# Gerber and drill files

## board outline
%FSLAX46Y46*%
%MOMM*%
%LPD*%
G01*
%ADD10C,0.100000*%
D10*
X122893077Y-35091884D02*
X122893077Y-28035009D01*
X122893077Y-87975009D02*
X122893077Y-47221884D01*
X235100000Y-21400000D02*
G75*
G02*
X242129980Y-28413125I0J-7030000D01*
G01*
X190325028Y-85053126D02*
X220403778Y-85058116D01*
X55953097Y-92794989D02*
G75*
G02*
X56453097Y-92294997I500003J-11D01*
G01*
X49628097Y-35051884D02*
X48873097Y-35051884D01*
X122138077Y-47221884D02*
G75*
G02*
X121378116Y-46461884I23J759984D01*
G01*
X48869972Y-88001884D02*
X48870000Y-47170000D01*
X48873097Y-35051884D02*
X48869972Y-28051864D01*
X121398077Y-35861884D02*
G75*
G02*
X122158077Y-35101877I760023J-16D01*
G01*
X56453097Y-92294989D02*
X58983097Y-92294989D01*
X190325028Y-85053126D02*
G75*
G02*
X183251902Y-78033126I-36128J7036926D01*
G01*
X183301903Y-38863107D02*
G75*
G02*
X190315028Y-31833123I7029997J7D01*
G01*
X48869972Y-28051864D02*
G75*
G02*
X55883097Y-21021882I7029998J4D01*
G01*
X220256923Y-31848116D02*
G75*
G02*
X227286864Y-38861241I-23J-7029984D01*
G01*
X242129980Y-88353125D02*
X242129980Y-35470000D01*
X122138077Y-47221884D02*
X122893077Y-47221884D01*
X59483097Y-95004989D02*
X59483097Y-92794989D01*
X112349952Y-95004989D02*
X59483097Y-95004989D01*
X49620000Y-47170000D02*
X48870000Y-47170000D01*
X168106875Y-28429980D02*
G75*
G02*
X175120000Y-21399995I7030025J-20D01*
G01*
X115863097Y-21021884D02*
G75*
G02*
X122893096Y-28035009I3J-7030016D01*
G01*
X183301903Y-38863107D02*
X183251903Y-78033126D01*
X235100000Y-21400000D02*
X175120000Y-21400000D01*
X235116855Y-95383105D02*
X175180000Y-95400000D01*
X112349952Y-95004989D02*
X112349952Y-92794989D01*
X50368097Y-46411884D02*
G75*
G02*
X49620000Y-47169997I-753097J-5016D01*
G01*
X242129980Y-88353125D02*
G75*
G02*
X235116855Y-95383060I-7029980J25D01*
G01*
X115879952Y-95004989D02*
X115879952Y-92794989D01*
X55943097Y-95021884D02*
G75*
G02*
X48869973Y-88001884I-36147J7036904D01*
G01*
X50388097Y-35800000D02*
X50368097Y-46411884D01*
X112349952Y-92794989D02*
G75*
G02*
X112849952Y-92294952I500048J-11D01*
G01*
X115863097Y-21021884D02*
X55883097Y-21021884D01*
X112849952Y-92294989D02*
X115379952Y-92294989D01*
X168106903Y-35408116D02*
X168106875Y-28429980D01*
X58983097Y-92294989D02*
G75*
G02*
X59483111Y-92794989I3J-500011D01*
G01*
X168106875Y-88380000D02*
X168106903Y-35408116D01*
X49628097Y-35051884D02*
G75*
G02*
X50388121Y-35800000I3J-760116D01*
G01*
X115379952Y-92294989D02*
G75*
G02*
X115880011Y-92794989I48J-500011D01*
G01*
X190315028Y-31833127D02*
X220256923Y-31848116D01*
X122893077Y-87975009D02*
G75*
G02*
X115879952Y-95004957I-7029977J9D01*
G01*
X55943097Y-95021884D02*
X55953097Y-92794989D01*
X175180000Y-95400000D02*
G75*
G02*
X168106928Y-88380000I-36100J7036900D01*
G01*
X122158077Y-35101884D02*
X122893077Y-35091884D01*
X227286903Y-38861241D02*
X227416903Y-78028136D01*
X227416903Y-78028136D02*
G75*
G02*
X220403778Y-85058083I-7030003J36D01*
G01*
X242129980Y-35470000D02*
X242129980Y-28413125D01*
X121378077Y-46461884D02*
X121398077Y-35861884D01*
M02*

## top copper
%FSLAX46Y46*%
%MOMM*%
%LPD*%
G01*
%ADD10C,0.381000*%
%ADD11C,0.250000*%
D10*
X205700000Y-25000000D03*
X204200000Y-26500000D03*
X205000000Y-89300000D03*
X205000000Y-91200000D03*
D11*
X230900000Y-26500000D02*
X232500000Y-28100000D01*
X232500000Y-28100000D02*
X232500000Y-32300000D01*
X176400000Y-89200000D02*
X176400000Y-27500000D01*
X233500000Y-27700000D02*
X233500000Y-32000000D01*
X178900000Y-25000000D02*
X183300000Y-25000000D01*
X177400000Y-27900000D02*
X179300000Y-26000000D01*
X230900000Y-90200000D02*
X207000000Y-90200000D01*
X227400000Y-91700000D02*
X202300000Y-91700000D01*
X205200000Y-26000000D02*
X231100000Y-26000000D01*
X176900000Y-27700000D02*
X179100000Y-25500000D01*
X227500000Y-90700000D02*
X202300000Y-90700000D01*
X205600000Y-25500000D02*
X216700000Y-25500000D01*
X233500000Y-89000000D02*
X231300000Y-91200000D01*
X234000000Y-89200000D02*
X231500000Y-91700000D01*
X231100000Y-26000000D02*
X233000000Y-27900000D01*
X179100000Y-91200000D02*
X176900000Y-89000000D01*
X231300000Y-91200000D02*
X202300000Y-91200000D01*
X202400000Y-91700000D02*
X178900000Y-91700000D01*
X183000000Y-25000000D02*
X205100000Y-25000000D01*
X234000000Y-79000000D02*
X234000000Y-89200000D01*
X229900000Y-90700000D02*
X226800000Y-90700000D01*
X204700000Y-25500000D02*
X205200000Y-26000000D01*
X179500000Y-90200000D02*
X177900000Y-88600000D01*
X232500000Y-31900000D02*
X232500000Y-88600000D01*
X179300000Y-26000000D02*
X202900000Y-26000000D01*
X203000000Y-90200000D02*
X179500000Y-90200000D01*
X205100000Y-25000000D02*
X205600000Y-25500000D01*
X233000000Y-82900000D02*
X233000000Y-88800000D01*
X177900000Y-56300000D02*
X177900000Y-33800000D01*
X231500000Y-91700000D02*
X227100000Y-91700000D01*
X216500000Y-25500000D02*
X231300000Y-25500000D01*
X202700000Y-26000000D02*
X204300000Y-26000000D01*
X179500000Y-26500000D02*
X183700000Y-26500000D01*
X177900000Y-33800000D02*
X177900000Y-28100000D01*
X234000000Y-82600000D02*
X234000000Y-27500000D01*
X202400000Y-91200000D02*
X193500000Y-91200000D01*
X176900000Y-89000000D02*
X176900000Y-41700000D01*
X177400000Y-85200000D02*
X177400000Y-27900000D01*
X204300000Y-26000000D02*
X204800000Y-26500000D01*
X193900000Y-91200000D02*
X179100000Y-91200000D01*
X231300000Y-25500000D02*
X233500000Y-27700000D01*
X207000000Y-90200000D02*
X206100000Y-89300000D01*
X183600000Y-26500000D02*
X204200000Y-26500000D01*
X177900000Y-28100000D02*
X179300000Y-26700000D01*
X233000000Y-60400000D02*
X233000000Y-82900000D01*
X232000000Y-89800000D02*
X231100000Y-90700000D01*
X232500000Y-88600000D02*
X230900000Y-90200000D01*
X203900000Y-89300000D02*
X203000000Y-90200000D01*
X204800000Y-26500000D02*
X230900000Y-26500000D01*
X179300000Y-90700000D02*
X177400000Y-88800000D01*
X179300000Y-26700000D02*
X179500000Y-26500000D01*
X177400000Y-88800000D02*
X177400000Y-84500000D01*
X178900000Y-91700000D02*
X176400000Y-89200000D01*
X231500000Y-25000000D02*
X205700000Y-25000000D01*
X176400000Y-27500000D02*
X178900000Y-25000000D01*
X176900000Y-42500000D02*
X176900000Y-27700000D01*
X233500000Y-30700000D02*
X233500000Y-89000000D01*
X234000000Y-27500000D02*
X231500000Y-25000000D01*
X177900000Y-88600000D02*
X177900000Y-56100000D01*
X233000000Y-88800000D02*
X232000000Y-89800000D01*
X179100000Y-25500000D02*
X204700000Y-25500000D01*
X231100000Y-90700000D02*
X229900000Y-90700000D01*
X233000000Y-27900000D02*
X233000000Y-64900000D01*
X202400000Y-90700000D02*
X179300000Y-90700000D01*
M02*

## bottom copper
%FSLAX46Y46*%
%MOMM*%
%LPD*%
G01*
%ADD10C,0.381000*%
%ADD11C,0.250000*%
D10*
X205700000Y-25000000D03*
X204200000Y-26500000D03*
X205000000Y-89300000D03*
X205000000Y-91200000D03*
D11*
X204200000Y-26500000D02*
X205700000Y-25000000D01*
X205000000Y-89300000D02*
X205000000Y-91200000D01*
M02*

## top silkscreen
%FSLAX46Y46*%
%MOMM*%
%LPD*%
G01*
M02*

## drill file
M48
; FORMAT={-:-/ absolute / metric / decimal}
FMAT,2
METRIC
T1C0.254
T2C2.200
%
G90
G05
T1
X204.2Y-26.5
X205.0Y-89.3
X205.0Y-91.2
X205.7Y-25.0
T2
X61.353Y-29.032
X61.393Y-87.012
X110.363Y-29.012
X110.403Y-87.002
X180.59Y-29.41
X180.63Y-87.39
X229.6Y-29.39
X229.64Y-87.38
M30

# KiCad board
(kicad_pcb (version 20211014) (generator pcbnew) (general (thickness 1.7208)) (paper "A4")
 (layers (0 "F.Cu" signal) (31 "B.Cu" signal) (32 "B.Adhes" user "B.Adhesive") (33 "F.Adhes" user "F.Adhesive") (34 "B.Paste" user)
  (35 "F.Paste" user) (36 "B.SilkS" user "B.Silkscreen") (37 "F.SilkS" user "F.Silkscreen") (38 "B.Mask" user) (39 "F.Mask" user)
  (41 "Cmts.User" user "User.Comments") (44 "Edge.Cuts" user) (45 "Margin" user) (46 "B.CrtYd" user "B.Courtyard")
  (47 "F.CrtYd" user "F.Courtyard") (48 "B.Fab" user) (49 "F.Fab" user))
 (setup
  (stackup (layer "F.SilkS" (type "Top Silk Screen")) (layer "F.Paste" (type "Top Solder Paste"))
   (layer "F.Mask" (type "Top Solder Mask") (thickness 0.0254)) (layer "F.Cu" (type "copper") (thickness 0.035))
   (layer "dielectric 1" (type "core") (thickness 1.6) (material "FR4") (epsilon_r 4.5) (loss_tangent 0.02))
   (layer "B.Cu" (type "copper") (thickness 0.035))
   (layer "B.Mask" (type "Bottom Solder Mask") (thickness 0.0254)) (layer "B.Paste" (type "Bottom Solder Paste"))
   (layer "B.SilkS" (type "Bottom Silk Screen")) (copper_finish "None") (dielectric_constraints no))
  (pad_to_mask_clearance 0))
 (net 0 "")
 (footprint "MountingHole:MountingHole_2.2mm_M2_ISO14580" (layer "F.Cu") (at 61.353097 29.031884)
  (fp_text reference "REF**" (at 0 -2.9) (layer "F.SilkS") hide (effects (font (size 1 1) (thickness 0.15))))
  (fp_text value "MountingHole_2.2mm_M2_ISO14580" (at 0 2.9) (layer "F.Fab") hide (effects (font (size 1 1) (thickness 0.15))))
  (pad "" np_thru_hole circle (at 0 0) (size 2.2 2.2) (drill 2.2) (layers *.Cu *.Mask)))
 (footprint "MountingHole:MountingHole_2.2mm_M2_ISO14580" (layer "F.Cu") (at 61.393097 87.011884)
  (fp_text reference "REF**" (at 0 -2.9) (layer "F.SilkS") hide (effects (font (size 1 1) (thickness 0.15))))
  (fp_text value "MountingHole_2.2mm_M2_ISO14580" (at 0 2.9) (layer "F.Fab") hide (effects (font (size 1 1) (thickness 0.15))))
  (pad "" np_thru_hole circle (at 0 0) (size 2.2 2.2) (drill 2.2) (layers *.Cu *.Mask)))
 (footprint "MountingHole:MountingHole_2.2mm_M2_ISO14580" (layer "F.Cu") (at 110.403097 87.001884)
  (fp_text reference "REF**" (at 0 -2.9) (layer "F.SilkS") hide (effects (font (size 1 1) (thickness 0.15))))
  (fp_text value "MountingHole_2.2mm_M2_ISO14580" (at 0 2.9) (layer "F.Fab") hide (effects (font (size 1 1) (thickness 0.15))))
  (pad "" np_thru_hole circle (at 0 0) (size 2.2 2.2) (drill 2.2) (layers *.Cu *.Mask)))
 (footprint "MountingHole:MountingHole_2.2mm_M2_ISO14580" (layer "F.Cu") (at 229.6 29.39)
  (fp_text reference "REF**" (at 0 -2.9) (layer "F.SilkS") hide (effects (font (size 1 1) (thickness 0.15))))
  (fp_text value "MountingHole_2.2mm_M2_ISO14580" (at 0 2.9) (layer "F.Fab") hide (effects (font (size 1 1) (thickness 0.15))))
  (pad "" np_thru_hole circle (at 0 0) (size 2.2 2.2) (drill 2.2) (layers *.Cu *.Mask)))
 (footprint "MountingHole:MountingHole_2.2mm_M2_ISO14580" (layer "F.Cu") (at 229.64 87.38)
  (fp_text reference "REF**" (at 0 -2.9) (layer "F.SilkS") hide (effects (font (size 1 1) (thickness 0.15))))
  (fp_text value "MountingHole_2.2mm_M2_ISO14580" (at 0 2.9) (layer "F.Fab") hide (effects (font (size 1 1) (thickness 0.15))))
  (pad "" np_thru_hole circle (at 0 0) (size 2.2 2.2) (drill 2.2) (layers *.Cu *.Mask)))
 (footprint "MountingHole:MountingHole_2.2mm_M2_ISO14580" (layer "F.Cu") (at 180.63 87.39)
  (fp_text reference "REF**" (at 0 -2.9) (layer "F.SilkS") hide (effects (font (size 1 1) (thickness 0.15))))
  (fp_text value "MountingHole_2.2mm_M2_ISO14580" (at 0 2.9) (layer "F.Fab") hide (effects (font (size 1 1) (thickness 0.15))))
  (pad "" np_thru_hole circle (at 0 0) (size 2.2 2.2) (drill 2.2) (layers *.Cu *.Mask)))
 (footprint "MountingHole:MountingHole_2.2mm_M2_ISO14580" (layer "F.Cu") (at 110.363097 29.011884)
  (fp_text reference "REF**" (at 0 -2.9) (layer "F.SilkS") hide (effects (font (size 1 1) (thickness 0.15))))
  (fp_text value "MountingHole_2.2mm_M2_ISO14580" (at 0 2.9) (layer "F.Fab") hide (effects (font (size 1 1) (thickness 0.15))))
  (pad "" np_thru_hole circle (at 0 0) (size 2.2 2.2) (drill 2.2) (layers *.Cu *.Mask)))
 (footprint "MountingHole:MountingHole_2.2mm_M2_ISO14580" (layer "F.Cu") (at 180.59 29.41)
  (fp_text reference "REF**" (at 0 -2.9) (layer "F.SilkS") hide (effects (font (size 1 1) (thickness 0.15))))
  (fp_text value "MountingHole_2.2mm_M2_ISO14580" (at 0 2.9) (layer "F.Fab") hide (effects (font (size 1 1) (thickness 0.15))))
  (pad "" np_thru_hole circle (at 0 0) (size 2.2 2.2) (drill 2.2) (layers *.Cu *.Mask)))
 (gr_line (start 122.893077 35.091884) (end 122.893077 28.035009) (layer "Edge.Cuts") (width 0.1))
 (gr_line (start 122.893077 87.975009) (end 122.893077 47.221884) (layer "Edge.Cuts") (width 0.1))
 (gr_arc (start 235.1 21.4) (mid 240.064991 23.453077) (end 242.12998 28.413125) (layer "Edge.Cuts") (width 0.1))
 (gr_line (start 190.325028 85.053126) (end 220.403778 85.058116) (layer "Edge.Cuts") (width 0.1))
 (gr_arc (start 55.953097 92.794989) (mid 56.099544 92.441436) (end 56.453097 92.294989) (layer "Edge.Cuts") (width 0.1))
 (gr_line (start 49.628097 35.051884) (end 48.873097 35.051884) (layer "Edge.Cuts") (width 0.1))
 (gr_arc (start 122.138077 47.221884) (mid 121.600676 46.999285) (end 121.378077 46.461884) (layer "Edge.Cuts") (width 0.1))
 (gr_line (start 48.869972 88.001884) (end 48.87 47.17) (layer "Edge.Cuts") (width 0.1))
 (gr_line (start 48.873097 35.051884) (end 48.869972 28.051864) (layer "Edge.Cuts") (width 0.1))
 (gr_arc (start 121.398077 35.861884) (mid 121.620676 35.324483) (end 122.158077 35.101884) (layer "Edge.Cuts") (width 0.1))
 (gr_line (start 56.453097 92.294989) (end 58.983097 92.294989) (layer "Edge.Cuts") (width 0.1))
 (gr_arc (start 190.325028 85.053126) (mid 185.331764 83.010851) (end 183.251903 78.033126) (layer "Edge.Cuts") (width 0.1))
 (gr_arc (start 183.301903 38.863107) (mid 185.35498 33.898116) (end 190.315028 31.833127) (layer "Edge.Cuts") (width 0.1))
 (gr_arc (start 48.869972 28.051864) (mid 50.923049 23.086873) (end 55.883097 21.021884) (layer "Edge.Cuts") (width 0.1))
 (gr_arc (start 220.256923 31.848116) (mid 225.221914 33.901193) (end 227.286903 38.861241) (layer "Edge.Cuts") (width 0.1))
 (gr_line (start 242.12998 88.353125) (end 242.12998 35.47) (layer "Edge.Cuts") (width 0.1))
 (gr_line (start 122.138077 47.221884) (end 122.893077 47.221884) (layer "Edge.Cuts") (width 0.1))
 (gr_line (start 59.483097 95.004989) (end 59.483097 92.794989) (layer "Edge.Cuts") (width 0.1))
 (gr_line (start 112.349952 95.004989) (end 59.483097 95.004989) (layer "Edge.Cuts") (width 0.1))
 (gr_line (start 49.62 47.17) (end 48.87 47.17) (layer "Edge.Cuts") (width 0.1))
 (gr_arc (start 168.106875 28.42998) (mid 170.159952 23.464989) (end 175.12 21.4) (layer "Edge.Cuts") (width 0.1))
 (gr_arc (start 115.863097 21.021884) (mid 120.828088 23.074961) (end 122.893077 28.035009) (layer "Edge.Cuts") (width 0.1))
 (gr_line (start 183.301903 38.863107) (end 183.251903 78.033126) (layer "Edge.Cuts") (width 0.1))
 (gr_line (start 235.1 21.4) (end 175.12 21.4) (layer "Edge.Cuts") (width 0.1))
 (gr_line (start 235.116855 95.383105) (end 175.18 95.4) (layer "Edge.Cuts") (width 0.1))
 (gr_line (start 112.349952 95.004989) (end 112.349952 92.794989) (layer "Edge.Cuts") (width 0.1))
 (gr_arc (start 50.368097 46.411884) (mid 50.15106 46.945878) (end 49.62 47.17) (layer "Edge.Cuts") (width 0.1))
 (gr_arc (start 242.12998 88.353125) (mid 240.076903 93.318116) (end 235.116855 95.383105) (layer "Edge.Cuts") (width 0.1))
 (gr_line (start 115.879952 95.004989) (end 115.879952 92.794989) (layer "Edge.Cuts") (width 0.1))
 (gr_arc (start 55.943097 95.021884) (mid 50.949833 92.979609) (end 48.869972 88.001884) (layer "Edge.Cuts") (width 0.1))
 (gr_line (start 50.388097 35.8) (end 50.368097 46.411884) (layer "Edge.Cuts") (width 0.1))
 (gr_arc (start 112.349952 92.794989) (mid 112.496399 92.441436) (end 112.849952 92.294989) (layer "Edge.Cuts") (width 0.1))
 (gr_line (start 115.863097 21.021884) (end 55.883097 21.021884) (layer "Edge.Cuts") (width 0.1))
 (gr_line (start 112.849952 92.294989) (end 115.379952 92.294989) (layer "Edge.Cuts") (width 0.1))
 (gr_line (start 168.106903 35.408116) (end 168.106875 28.42998) (layer "Edge.Cuts") (width 0.1))
 (gr_arc (start 58.983097 92.294989) (mid 59.33665 92.441436) (end 59.483097 92.794989) (layer "Edge.Cuts") (width 0.1))
 (gr_line (start 168.106875 88.38) (end 168.106903 35.408116) (layer "Edge.Cuts") (width 0.1))
 (gr_arc (start 49.628097 35.051884) (mid 50.161313 35.270292) (end 50.388097 35.8) (layer "Edge.Cuts") (width 0.1))
 (gr_arc (start 115.379952 92.294989) (mid 115.733505 92.441436) (end 115.879952 92.794989) (layer "Edge.Cuts") (width 0.1))
 (gr_line (start 190.315028 31.833127) (end 220.256923 31.848116) (layer "Edge.Cuts") (width 0.1))
 (gr_arc (start 122.893077 87.975009) (mid 120.84 92.94) (end 115.879952 95.004989) (layer "Edge.Cuts") (width 0.1))
 (gr_line (start 55.943097 95.021884) (end 55.953097 92.794989) (layer "Edge.Cuts") (width 0.1))
 (gr_arc (start 175.18 95.4) (mid 170.186736 93.357725) (end 168.106875 88.38) (layer "Edge.Cuts") (width 0.1))
 (gr_line (start 122.158077 35.101884) (end 122.893077 35.091884) (layer "Edge.Cuts") (width 0.1))
 (gr_line (start 227.286903 38.861241) (end 227.416903 78.028136) (layer "Edge.Cuts") (width 0.1))
 (gr_arc (start 227.416903 78.028136) (mid 225.363826 82.993127) (end 220.403778 85.058116) (layer "Edge.Cuts") (width 0.1))
 (gr_line (start 242.12998 35.47) (end 242.12998 28.413125) (layer "Edge.Cuts") (width 0.1))
 (gr_line (start 121.378077 46.461884) (end 121.398077 35.861884) (layer "Edge.Cuts") (width 0.1))
 (segment (start 230.9 26.5) (end 232.5 28.1) (width 0.25) (layer "F.Cu") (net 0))
 (segment (start 232.5 28.1) (end 232.5 32.3) (width 0.25) (layer "F.Cu") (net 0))
 (segment (start 176.4 89.2) (end 176.4 27.5) (width 0.25) (layer "F.Cu") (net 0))
 (segment (start 233.5 27.7) (end 233.5 32) (width 0.25) (layer "F.Cu") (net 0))
 (segment (start 178.9 25) (end 183.3 25) (width 0.25) (layer "F.Cu") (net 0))
 (segment (start 177.4 27.9) (end 179.3 26) (width 0.25) (layer "F.Cu") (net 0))
 (segment (start 230.9 90.2) (end 207 90.2) (width 0.25) (layer "F.Cu") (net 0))
 (segment (start 227.4 91.7) (end 202.3 91.7) (width 0.25) (layer "F.Cu") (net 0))
 (segment (start 205.2 26) (end 231.1 26) (width 0.25) (layer "F.Cu") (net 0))
 (segment (start 176.9 27.7) (end 179.1 25.5) (width 0.25) (layer "F.Cu") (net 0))
 (segment (start 227.5 90.7) (end 202.3 90.7) (width 0.25) (layer "F.Cu") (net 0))
 (segment (start 205.6 25.5) (end 216.7 25.5) (width 0.25) (layer "F.Cu") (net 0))
 (segment (start 233.5 89) (end 231.3 91.2) (width 0.25) (layer "F.Cu") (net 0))
 (segment (start 234 89.2) (end 231.5 91.7) (width 0.25) (layer "F.Cu") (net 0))
 (segment (start 231.1 26) (end 233 27.9) (width 0.25) (layer "F.Cu") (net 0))
 (segment (start 179.1 91.2) (end 176.9 89) (width 0.25) (layer "F.Cu") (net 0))
 (segment (start 231.3 91.2) (end 202.3 91.2) (width 0.25) (layer "F.Cu") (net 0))
 (segment (start 202.4 91.7) (end 178.9 91.7) (width 0.25) (layer "F.Cu") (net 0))
 (segment (start 183 25) (end 205.1 25) (width 0.25) (layer "F.Cu") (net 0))
 (segment (start 234 79) (end 234 89.2) (width 0.25) (layer "F.Cu") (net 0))
 (segment (start 229.9 90.7) (end 226.8 90.7) (width 0.25) (layer "F.Cu") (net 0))
 (segment (start 204.7 25.5) (end 205.2 26) (width 0.25) (layer "F.Cu") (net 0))
 (segment (start 179.5 90.2) (end 177.9 88.6) (width 0.25) (layer "F.Cu") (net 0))
 (segment (start 232.5 31.9) (end 232.5 88.6) (width 0.25) (layer "F.Cu") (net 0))
 (segment (start 179.3 26) (end 202.9 26) (width 0.25) (layer "F.Cu") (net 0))
 (segment (start 203 90.2) (end 179.5 90.2) (width 0.25) (layer "F.Cu") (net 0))
 (segment (start 205.1 25) (end 205.6 25.5) (width 0.25) (layer "F.Cu") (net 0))
 (segment (start 233 82.9) (end 233 88.8) (width 0.25) (layer "F.Cu") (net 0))
 (segment (start 177.9 56.3) (end 177.9 33.8) (width 0.25) (layer "F.Cu") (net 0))
 (segment (start 231.5 91.7) (end 227.1 91.7) (width 0.25) (layer "F.Cu") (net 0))
 (segment (start 216.5 25.5) (end 231.3 25.5) (width 0.25) (layer "F.Cu") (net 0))
 (segment (start 202.7 26) (end 204.3 26) (width 0.25) (layer "F.Cu") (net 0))
 (segment (start 179.5 26.5) (end 183.7 26.5) (width 0.25) (layer "F.Cu") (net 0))
 (segment (start 177.9 33.8) (end 177.9 28.1) (width 0.25) (layer "F.Cu") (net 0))
 (segment (start 234 82.6) (end 234 27.5) (width 0.25) (layer "F.Cu") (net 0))
 (segment (start 202.4 91.2) (end 193.5 91.2) (width 0.25) (layer "F.Cu") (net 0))
 (segment (start 176.9 89) (end 176.9 41.7) (width 0.25) (layer "F.Cu") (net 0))
 (segment (start 177.4 85.2) (end 177.4 27.9) (width 0.25) (layer "F.Cu") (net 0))
 (segment (start 204.3 26) (end 204.8 26.5) (width 0.25) (layer "F.Cu") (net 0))
 (segment (start 193.9 91.2) (end 179.1 91.2) (width 0.25) (layer "F.Cu") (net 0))
 (segment (start 231.3 25.5) (end 233.5 27.7) (width 0.25) (layer "F.Cu") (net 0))
 (segment (start 207 90.2) (end 206.1 89.3) (width 0.25) (layer "F.Cu") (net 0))
 (segment (start 183.6 26.5) (end 204.2 26.5) (width 0.25) (layer "F.Cu") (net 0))
 (segment (start 177.9 28.1) (end 179.3 26.7) (width 0.25) (layer "F.Cu") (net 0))
 (segment (start 233 60.4) (end 233 82.9) (width 0.25) (layer "F.Cu") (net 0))
 (segment (start 232 89.8) (end 231.1 90.7) (width 0.25) (layer "F.Cu") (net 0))
 (segment (start 232.5 88.6) (end 230.9 90.2) (width 0.25) (layer "F.Cu") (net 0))
 (segment (start 203.9 89.3) (end 203 90.2) (width 0.25) (layer "F.Cu") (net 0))
 (segment (start 204.8 26.5) (end 230.9 26.5) (width 0.25) (layer "F.Cu") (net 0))
 (segment (start 179.3 90.7) (end 177.4 88.8) (width 0.25) (layer "F.Cu") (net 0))
 (segment (start 179.3 26.7) (end 179.5 26.5) (width 0.25) (layer "F.Cu") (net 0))
 (segment (start 177.4 88.8) (end 177.4 84.5) (width 0.25) (layer "F.Cu") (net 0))
 (segment (start 178.9 91.7) (end 176.4 89.2) (width 0.25) (layer "F.Cu") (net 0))
 (segment (start 231.5 25) (end 205.7 25) (width 0.25) (layer "F.Cu") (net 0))
 (segment (start 176.4 27.5) (end 178.9 25) (width 0.25) (layer "F.Cu") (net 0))
 (segment (start 176.9 42.5) (end 176.9 27.7) (width 0.25) (layer "F.Cu") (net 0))
 (segment (start 233.5 30.7) (end 233.5 89) (width 0.25) (layer "F.Cu") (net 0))
 (segment (start 234 27.5) (end 231.5 25) (width 0.25) (layer "F.Cu") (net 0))
 (segment (start 177.9 88.6) (end 177.9 56.1) (width 0.25) (layer "F.Cu") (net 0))
 (segment (start 233 88.8) (end 232 89.8) (width 0.25) (layer "F.Cu") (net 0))
 (segment (start 179.1 25.5) (end 204.7 25.5) (width 0.25) (layer "F.Cu") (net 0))
 (segment (start 231.1 90.7) (end 229.9 90.7) (width 0.25) (layer "F.Cu") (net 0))
 (segment (start 233 27.9) (end 233 64.9) (width 0.25) (layer "F.Cu") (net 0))
 (segment (start 202.4 90.7) (end 179.3 90.7) (width 0.25) (layer "F.Cu") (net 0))
 (via (at 205.7 25) (size 0.381) (drill 0.254) (layers "F.Cu" "B.Cu") (free) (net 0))
 (via (at 204.2 26.5) (size 0.381) (drill 0.254) (layers "F.Cu" "B.Cu") (free) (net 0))
 (via (at 205 89.3) (size 0.381) (drill 0.254) (layers "F.Cu" "B.Cu") (free) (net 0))
 (via (at 205 91.2) (size 0.381) (drill 0.254) (layers "F.Cu" "B.Cu") (free) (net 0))
 (segment (start 204.2 26.5) (end 205.7 25) (width 0.25) (layer "B.Cu") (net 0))
 (segment (start 205 89.3) (end 205 91.2) (width 0.25) (layer "B.Cu") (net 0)))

